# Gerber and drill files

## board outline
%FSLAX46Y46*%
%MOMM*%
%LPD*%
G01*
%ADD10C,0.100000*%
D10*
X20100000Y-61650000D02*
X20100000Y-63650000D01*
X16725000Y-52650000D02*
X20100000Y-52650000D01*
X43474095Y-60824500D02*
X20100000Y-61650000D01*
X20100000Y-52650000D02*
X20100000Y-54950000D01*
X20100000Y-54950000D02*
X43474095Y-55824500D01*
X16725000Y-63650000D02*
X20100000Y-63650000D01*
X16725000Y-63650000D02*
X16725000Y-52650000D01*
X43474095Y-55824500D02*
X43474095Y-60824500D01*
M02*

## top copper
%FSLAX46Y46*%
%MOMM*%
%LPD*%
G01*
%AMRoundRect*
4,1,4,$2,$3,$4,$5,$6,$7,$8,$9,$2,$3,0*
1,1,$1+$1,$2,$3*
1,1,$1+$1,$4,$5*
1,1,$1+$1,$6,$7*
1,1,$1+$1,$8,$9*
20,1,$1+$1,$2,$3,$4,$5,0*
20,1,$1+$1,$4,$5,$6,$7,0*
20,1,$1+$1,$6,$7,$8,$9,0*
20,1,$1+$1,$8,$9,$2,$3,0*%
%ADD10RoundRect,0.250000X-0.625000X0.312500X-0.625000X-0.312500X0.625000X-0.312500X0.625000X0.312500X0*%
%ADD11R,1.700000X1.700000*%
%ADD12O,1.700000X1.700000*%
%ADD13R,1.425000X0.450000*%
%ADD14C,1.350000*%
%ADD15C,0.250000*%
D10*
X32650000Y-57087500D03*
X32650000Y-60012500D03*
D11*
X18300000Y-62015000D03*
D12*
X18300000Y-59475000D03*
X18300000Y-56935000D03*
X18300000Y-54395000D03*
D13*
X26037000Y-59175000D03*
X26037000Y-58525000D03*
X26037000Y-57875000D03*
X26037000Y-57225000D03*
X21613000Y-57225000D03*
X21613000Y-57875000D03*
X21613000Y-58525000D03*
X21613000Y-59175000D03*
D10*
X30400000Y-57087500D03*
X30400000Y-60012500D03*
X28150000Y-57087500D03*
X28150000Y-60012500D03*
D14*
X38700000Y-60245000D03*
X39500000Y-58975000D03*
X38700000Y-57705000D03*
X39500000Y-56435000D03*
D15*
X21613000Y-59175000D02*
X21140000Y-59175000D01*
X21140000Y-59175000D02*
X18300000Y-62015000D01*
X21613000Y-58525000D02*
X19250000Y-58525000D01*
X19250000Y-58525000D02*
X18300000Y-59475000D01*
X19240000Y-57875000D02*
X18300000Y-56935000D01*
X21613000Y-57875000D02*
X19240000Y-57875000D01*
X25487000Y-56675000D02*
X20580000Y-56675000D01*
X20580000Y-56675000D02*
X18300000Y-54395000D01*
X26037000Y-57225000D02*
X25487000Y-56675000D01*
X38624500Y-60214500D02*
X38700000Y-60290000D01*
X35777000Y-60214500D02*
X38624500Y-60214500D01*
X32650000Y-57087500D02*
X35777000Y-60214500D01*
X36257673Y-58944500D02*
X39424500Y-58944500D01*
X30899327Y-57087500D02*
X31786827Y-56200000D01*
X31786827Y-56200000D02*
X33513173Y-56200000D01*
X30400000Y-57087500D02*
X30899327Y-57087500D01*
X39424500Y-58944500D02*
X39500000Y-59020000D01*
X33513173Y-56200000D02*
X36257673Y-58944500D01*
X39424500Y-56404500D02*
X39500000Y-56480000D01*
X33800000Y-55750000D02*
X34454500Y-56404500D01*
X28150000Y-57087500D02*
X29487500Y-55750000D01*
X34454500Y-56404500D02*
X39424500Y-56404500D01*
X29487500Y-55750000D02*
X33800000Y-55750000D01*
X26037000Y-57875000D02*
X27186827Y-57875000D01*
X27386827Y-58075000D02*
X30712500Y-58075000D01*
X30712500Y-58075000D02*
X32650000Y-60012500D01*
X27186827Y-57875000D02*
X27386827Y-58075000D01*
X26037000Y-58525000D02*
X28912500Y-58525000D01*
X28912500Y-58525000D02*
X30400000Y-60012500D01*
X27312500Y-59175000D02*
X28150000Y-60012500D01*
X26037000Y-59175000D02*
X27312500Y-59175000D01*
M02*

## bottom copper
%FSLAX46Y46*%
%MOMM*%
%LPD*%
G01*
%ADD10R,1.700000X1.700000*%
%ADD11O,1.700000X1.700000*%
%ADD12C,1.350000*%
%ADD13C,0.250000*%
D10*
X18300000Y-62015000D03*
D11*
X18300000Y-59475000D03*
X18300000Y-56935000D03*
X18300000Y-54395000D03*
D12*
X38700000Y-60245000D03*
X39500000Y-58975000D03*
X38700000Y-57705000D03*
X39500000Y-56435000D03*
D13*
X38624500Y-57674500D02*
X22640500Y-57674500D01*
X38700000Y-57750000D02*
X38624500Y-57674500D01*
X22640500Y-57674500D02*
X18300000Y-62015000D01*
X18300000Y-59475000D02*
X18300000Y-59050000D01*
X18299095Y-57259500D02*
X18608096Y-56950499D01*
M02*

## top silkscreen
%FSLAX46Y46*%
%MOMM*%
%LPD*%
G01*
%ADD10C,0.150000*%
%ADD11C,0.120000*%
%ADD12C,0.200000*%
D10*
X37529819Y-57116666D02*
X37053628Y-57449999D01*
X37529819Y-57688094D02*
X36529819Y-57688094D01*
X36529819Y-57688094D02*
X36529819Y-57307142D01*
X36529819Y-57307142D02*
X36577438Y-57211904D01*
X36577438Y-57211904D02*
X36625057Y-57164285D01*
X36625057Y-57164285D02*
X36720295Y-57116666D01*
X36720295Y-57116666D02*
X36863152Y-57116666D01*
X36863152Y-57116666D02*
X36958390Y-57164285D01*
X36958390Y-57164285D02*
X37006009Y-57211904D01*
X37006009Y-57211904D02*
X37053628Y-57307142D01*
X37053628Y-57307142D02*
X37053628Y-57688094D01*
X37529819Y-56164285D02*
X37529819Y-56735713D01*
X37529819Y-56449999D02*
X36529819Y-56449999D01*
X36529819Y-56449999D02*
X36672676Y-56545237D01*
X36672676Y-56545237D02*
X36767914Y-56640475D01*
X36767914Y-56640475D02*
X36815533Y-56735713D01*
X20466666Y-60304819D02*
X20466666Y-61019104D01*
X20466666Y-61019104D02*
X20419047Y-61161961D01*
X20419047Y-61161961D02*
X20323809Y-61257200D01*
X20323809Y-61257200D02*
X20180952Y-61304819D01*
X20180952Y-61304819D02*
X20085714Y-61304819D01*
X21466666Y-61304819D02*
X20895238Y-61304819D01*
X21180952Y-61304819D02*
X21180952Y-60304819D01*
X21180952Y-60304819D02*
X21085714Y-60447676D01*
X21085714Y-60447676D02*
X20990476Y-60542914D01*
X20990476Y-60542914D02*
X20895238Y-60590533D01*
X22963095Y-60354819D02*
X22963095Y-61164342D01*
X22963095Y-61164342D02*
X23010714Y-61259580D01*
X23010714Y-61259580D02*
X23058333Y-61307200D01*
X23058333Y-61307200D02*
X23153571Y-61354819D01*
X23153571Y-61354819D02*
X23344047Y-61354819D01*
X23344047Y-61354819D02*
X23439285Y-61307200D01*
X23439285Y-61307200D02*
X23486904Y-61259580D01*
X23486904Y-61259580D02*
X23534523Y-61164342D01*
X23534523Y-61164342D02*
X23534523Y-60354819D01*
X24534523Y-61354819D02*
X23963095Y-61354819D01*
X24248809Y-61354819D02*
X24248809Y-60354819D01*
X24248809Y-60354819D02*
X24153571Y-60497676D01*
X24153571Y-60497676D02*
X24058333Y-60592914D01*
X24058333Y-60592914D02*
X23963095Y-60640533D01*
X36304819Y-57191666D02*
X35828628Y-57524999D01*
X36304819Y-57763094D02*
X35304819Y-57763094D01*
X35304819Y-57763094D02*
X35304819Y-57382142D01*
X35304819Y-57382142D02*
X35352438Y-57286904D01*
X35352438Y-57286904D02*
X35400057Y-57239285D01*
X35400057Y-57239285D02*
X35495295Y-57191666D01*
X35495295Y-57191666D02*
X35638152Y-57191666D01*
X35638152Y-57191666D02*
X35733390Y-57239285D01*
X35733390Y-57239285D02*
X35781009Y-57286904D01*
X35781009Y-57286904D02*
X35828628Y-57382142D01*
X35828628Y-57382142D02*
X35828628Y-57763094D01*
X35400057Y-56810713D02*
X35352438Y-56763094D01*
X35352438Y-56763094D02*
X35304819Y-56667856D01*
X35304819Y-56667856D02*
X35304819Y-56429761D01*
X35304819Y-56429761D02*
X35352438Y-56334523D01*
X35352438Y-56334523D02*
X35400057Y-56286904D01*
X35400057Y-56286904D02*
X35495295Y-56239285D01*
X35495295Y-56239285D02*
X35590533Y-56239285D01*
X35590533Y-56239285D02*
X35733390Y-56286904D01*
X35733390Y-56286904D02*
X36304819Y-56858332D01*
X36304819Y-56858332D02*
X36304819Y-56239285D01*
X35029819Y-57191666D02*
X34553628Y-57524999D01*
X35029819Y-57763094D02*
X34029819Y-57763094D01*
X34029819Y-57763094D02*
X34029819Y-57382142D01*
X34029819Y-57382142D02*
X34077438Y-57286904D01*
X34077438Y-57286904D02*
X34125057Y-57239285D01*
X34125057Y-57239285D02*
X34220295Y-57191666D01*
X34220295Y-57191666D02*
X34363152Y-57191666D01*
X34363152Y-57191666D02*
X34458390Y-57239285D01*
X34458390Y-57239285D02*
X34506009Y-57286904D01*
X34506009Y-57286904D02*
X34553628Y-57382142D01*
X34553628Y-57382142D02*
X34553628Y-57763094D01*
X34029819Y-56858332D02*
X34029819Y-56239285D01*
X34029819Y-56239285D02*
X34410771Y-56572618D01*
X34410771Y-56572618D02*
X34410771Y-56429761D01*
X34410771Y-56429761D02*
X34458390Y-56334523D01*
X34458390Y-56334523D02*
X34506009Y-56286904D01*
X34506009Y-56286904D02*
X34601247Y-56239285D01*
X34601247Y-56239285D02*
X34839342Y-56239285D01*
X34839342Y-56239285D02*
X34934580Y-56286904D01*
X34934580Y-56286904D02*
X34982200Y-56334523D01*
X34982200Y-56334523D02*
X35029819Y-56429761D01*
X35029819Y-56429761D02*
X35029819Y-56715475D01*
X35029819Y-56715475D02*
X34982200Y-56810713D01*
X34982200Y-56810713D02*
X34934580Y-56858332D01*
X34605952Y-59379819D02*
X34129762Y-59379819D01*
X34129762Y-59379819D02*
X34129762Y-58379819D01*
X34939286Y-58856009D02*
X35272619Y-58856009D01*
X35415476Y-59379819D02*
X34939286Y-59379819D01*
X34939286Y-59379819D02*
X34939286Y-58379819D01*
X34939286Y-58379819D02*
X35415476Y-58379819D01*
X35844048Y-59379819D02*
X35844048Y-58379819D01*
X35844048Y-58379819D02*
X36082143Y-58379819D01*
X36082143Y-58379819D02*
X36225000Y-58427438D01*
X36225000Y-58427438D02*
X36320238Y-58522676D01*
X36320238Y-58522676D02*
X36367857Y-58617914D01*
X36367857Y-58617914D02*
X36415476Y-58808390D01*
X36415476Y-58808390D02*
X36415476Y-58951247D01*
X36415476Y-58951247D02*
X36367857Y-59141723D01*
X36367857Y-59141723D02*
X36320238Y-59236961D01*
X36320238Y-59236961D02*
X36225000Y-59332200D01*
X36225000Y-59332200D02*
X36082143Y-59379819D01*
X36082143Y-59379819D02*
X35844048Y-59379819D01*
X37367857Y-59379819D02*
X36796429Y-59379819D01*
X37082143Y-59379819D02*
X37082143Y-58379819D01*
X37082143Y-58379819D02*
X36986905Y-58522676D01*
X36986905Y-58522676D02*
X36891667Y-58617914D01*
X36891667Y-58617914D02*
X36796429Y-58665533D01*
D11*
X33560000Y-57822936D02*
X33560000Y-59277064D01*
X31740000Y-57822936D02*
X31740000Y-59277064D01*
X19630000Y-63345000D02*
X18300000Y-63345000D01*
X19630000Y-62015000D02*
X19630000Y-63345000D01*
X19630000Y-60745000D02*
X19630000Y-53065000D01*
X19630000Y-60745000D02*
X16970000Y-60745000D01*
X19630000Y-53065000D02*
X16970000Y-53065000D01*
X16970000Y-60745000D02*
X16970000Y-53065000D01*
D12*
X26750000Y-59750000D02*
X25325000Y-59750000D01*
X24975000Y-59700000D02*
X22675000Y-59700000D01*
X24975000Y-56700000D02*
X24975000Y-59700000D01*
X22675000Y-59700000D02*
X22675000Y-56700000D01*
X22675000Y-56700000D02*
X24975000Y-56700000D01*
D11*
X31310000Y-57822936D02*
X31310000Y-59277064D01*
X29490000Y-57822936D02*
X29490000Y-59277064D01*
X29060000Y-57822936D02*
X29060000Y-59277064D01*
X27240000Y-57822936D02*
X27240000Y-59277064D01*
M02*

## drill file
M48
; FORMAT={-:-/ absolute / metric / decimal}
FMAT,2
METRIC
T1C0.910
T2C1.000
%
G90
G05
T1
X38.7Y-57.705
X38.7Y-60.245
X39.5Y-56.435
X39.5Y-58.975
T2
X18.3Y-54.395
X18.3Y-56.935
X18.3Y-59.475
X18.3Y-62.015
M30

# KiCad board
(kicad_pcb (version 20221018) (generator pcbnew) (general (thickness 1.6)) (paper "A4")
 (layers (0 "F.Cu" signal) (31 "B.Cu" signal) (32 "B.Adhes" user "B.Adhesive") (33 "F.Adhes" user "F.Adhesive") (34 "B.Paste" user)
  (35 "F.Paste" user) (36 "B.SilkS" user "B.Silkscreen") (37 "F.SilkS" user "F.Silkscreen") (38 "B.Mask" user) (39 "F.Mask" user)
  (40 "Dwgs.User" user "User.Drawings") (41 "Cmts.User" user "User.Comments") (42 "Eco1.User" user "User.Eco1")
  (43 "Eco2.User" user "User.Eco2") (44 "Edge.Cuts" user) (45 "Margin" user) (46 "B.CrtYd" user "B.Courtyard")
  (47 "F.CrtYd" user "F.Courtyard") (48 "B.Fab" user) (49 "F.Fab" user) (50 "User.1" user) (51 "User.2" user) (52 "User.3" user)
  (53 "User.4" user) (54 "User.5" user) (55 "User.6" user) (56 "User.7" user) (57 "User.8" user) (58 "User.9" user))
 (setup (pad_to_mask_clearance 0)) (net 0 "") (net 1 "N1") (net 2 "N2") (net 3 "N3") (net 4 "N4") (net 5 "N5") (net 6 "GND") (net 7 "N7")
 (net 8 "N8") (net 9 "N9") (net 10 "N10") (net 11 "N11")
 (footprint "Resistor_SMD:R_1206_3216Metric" (layer "F.Cu") (at 32.65 58.55 -90)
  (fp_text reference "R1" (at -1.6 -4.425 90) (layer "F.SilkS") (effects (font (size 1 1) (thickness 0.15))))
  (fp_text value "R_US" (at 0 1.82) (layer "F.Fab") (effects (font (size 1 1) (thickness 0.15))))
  (fp_line (start -0.727064 -0.91) (end 0.727064 -0.91) (stroke (width 0.12) (type solid)) (layer "F.SilkS"))
  (fp_line (start -0.727064 0.91) (end 0.727064 0.91) (stroke (width 0.12) (type solid)) (layer "F.SilkS"))
  (pad "1" smd roundrect (at -1.4625 0 270) (size 1.125 1.75) (layers "F.Cu" "F.Paste" "F.Mask") (roundrect_rratio 0.2222222222)
   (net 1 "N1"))
  (pad "2" smd roundrect (at 1.4625 0 270) (size 1.125 1.75) (layers "F.Cu" "F.Paste" "F.Mask") (roundrect_rratio 0.2222222222) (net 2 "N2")))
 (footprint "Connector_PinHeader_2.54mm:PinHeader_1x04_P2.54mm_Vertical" (layer "F.Cu") (at 18.3 62.015 180)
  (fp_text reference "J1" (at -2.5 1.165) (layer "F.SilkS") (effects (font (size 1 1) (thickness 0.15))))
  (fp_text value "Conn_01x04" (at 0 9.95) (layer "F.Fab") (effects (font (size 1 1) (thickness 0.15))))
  (fp_line (start -1.33 -1.33) (end 0 -1.33) (stroke (width 0.12) (type solid)) (layer "F.SilkS"))
  (fp_line (start -1.33 0) (end -1.33 -1.33) (stroke (width 0.12) (type solid)) (layer "F.SilkS"))
  (fp_line (start -1.33 1.27) (end -1.33 8.95) (stroke (width 0.12) (type solid)) (layer "F.SilkS"))
  (fp_line (start -1.33 1.27) (end 1.33 1.27) (stroke (width 0.12) (type solid)) (layer "F.SilkS"))
  (fp_line (start -1.33 8.95) (end 1.33 8.95) (stroke (width 0.12) (type solid)) (layer "F.SilkS"))
  (fp_line (start 1.33 1.27) (end 1.33 8.95) (stroke (width 0.12) (type solid)) (layer "F.SilkS"))
  (pad "1" thru_hole rect (at 0 0 180) (size 1.7 1.7) (drill 1) (layers "*.Cu" "*.Mask") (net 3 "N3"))
  (pad "2" thru_hole oval (at 0 2.54 180) (size 1.7 1.7) (drill 1) (layers "*.Cu" "*.Mask") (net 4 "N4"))
  (pad "3" thru_hole oval (at 0 5.08 180) (size 1.7 1.7) (drill 1) (layers "*.Cu" "*.Mask") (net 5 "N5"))
  (pad "4" thru_hole oval (at 0 7.62 180) (size 1.7 1.7) (drill 1) (layers "*.Cu" "*.Mask") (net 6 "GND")))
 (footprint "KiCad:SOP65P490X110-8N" (layer "F.Cu") (at 23.825 58.2 180)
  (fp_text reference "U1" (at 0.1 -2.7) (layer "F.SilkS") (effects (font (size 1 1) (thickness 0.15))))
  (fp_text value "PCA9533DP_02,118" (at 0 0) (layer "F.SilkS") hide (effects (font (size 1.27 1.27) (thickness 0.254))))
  (fp_line (start -2.925 -1.55) (end -1.5 -1.55) (stroke (width 0.2) (type solid)) (layer "F.SilkS"))
  (fp_line (start -1.15 -1.5) (end 1.15 -1.5) (stroke (width 0.2) (type solid)) (layer "F.SilkS"))
  (fp_line (start -1.15 1.5) (end -1.15 -1.5) (stroke (width 0.2) (type solid)) (layer "F.SilkS"))
  (fp_line (start 1.15 -1.5) (end 1.15 1.5) (stroke (width 0.2) (type solid)) (layer "F.SilkS"))
  (fp_line (start 1.15 1.5) (end -1.15 1.5) (stroke (width 0.2) (type solid)) (layer "F.SilkS"))
  (pad "1" smd rect (at -2.212 -0.975 270) (size 0.45 1.425) (layers "F.Cu" "F.Paste" "F.Mask") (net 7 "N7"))
  (pad "2" smd rect (at -2.212 -0.325 270) (size 0.45 1.425) (layers "F.Cu" "F.Paste" "F.Mask") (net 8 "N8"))
  (pad "3" smd rect (at -2.212 0.325 270) (size 0.45 1.425) (layers "F.Cu" "F.Paste" "F.Mask") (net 2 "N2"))
  (pad "4" smd rect (at -2.212 0.975 270) (size 0.45 1.425) (layers "F.Cu" "F.Paste" "F.Mask") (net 6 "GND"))
  (pad "5" smd rect (at 2.212 0.975 270) (size 0.45 1.425) (layers "F.Cu" "F.Paste" "F.Mask") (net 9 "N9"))
  (pad "6" smd rect (at 2.212 0.325 270) (size 0.45 1.425) (layers "F.Cu" "F.Paste" "F.Mask") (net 5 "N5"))
  (pad "7" smd rect (at 2.212 -0.325 270) (size 0.45 1.425) (layers "F.Cu" "F.Paste" "F.Mask") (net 4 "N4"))
  (pad "8" smd rect (at 2.212 -0.975 270) (size 0.45 1.425) (layers "F.Cu" "F.Paste" "F.Mask") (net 3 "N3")))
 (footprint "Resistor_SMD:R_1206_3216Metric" (layer "F.Cu") (at 30.4 58.55 -90)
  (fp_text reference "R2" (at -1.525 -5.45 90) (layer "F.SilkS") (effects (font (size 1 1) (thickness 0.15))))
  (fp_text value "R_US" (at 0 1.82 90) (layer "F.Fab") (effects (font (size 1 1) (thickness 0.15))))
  (fp_line (start -0.727064 -0.91) (end 0.727064 -0.91) (stroke (width 0.12) (type solid)) (layer "F.SilkS"))
  (fp_line (start -0.727064 0.91) (end 0.727064 0.91) (stroke (width 0.12) (type solid)) (layer "F.SilkS"))
  (pad "1" smd roundrect (at -1.4625 0 270) (size 1.125 1.75) (layers "F.Cu" "F.Paste" "F.Mask") (roundrect_rratio 0.2222222222)
   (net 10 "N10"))
  (pad "2" smd roundrect (at 1.4625 0 270) (size 1.125 1.75) (layers "F.Cu" "F.Paste" "F.Mask") (roundrect_rratio 0.2222222222) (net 8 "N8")))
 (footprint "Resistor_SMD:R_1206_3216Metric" (layer "F.Cu") (at 28.15 58.55 -90)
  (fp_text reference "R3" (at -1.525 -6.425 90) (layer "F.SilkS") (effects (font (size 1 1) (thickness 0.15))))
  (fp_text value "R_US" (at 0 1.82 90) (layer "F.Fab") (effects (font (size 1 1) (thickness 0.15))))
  (fp_line (start -0.727064 -0.91) (end 0.727064 -0.91) (stroke (width 0.12) (type solid)) (layer "F.SilkS"))
  (fp_line (start -0.727064 0.91) (end 0.727064 0.91) (stroke (width 0.12) (type solid)) (layer "F.SilkS"))
  (pad "1" smd roundrect (at -1.4625 0 270) (size 1.125 1.75) (layers "F.Cu" "F.Paste" "F.Mask") (roundrect_rratio 0.2222222222)
   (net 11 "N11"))
  (pad "2" smd roundrect (at 1.4625 0 270) (size 1.125 1.75) (layers "F.Cu" "F.Paste" "F.Mask") (roundrect_rratio 0.2222222222) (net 7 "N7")))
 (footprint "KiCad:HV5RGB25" (layer "F.Cu") (at 38.7 60.245 90)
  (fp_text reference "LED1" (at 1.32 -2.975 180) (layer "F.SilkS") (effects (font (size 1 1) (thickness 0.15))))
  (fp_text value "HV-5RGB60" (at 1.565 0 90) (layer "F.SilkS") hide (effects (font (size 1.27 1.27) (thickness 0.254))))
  (pad "1" thru_hole circle (at 0 0 90) (size 1.35 1.35) (drill 0.91) (layers "*.Cu" "*.Mask") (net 1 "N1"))
  (pad "2" thru_hole circle (at 1.27 0.8 90) (size 1.35 1.35) (drill 0.91) (layers "*.Cu" "*.Mask") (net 10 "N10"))
  (pad "3" thru_hole circle (at 2.54 0 90) (size 1.35 1.35) (drill 0.91) (layers "*.Cu" "*.Mask") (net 3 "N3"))
  (pad "4" thru_hole circle (at 3.81 0.8 90) (size 1.35 1.35) (drill 0.91) (layers "*.Cu" "*.Mask") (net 11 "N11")))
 (gr_line (start 20.1 61.65) (end 20.1 63.65) (stroke (width 0.1) (type default)) (layer "Edge.Cuts"))
 (gr_line (start 16.725 52.65) (end 20.1 52.65) (stroke (width 0.1) (type default)) (layer "Edge.Cuts"))
 (gr_line (start 43.474095 60.8245) (end 20.1 61.65) (stroke (width 0.1) (type default)) (layer "Edge.Cuts"))
 (gr_line (start 20.1 52.65) (end 20.1 54.95) (stroke (width 0.1) (type default)) (layer "Edge.Cuts"))
 (gr_line (start 20.1 54.95) (end 43.474095 55.8245) (stroke (width 0.1) (type default)) (layer "Edge.Cuts"))
 (gr_line (start 16.725 63.65) (end 20.1 63.65) (stroke (width 0.1) (type default)) (layer "Edge.Cuts"))
 (gr_line (start 16.725 63.65) (end 16.725 52.65) (stroke (width 0.1) (type default)) (layer "Edge.Cuts"))
 (gr_line (start 43.474095 55.8245) (end 43.474095 60.8245) (stroke (width 0.1) (type default)) (layer "Edge.Cuts"))
 (segment (start 21.613 59.175) (end 21.14 59.175) (width 0.25) (layer "F.Cu") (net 3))
 (segment (start 21.14 59.175) (end 18.3 62.015) (width 0.25) (layer "F.Cu") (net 3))
 (segment (start 38.6245 57.6745) (end 22.6405 57.6745) (width 0.25) (layer "B.Cu") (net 3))
 (segment (start 38.7 57.75) (end 38.6245 57.6745) (width 0.25) (layer "B.Cu") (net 3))
 (segment (start 22.6405 57.6745) (end 18.3 62.015) (width 0.25) (layer "B.Cu") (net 3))
 (segment (start 21.613 58.525) (end 19.25 58.525) (width 0.25) (layer "F.Cu") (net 4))
 (segment (start 19.25 58.525) (end 18.3 59.475) (width 0.25) (layer "F.Cu") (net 4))
 (segment (start 18.3 59.475) (end 18.3 59.05) (width 0.25) (layer "B.Cu") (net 4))
 (segment (start 19.24 57.875) (end 18.3 56.935) (width 0.25) (layer "F.Cu") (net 5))
 (segment (start 21.613 57.875) (end 19.24 57.875) (width 0.25) (layer "F.Cu") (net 5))
 (segment (start 18.299095 57.2595) (end 18.608096 56.950499) (width 0.25) (layer "B.Cu") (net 5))
 (segment (start 25.487 56.675) (end 20.58 56.675) (width 0.25) (layer "F.Cu") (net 6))
 (segment (start 20.58 56.675) (end 18.3 54.395) (width 0.25) (layer "F.Cu") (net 6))
 (segment (start 26.037 57.225) (end 25.487 56.675) (width 0.25) (layer "F.Cu") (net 6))
 (segment (start 38.6245 60.2145) (end 38.7 60.29) (width 0.25) (layer "F.Cu") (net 1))
 (segment (start 35.777 60.2145) (end 38.6245 60.2145) (width 0.25) (layer "F.Cu") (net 1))
 (segment (start 32.65 57.0875) (end 35.777 60.2145) (width 0.25) (layer "F.Cu") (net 1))
 (segment (start 36.257673 58.9445) (end 39.4245 58.9445) (width 0.25) (layer "F.Cu") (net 10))
 (segment (start 30.899327 57.0875) (end 31.786827 56.2) (width 0.25) (layer "F.Cu") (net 10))
 (segment (start 31.786827 56.2) (end 33.513173 56.2) (width 0.25) (layer "F.Cu") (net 10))
 (segment (start 30.4 57.0875) (end 30.899327 57.0875) (width 0.25) (layer "F.Cu") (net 10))
 (segment (start 39.4245 58.9445) (end 39.5 59.02) (width 0.25) (layer "F.Cu") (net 10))
 (segment (start 33.513173 56.2) (end 36.257673 58.9445) (width 0.25) (layer "F.Cu") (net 10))
 (segment (start 39.4245 56.4045) (end 39.5 56.48) (width 0.25) (layer "F.Cu") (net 11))
 (segment (start 33.8 55.75) (end 34.4545 56.4045) (width 0.25) (layer "F.Cu") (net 11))
 (segment (start 28.15 57.0875) (end 29.4875 55.75) (width 0.25) (layer "F.Cu") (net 11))
 (segment (start 34.4545 56.4045) (end 39.4245 56.4045) (width 0.25) (layer "F.Cu") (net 11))
 (segment (start 29.4875 55.75) (end 33.8 55.75) (width 0.25) (layer "F.Cu") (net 11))
 (segment (start 26.037 57.875) (end 27.186827 57.875) (width 0.25) (layer "F.Cu") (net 2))
 (segment (start 27.386827 58.075) (end 30.7125 58.075) (width 0.25) (layer "F.Cu") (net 2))
 (segment (start 30.7125 58.075) (end 32.65 60.0125) (width 0.25) (layer "F.Cu") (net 2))
 (segment (start 27.186827 57.875) (end 27.386827 58.075) (width 0.25) (layer "F.Cu") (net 2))
 (segment (start 26.037 58.525) (end 28.9125 58.525) (width 0.25) (layer "F.Cu") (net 8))
 (segment (start 28.9125 58.525) (end 30.4 60.0125) (width 0.25) (layer "F.Cu") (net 8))
 (segment (start 27.3125 59.175) (end 28.15 60.0125) (width 0.25) (layer "F.Cu") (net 7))
 (segment (start 26.037 59.175) (end 27.3125 59.175) (width 0.25) (layer "F.Cu") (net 7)))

